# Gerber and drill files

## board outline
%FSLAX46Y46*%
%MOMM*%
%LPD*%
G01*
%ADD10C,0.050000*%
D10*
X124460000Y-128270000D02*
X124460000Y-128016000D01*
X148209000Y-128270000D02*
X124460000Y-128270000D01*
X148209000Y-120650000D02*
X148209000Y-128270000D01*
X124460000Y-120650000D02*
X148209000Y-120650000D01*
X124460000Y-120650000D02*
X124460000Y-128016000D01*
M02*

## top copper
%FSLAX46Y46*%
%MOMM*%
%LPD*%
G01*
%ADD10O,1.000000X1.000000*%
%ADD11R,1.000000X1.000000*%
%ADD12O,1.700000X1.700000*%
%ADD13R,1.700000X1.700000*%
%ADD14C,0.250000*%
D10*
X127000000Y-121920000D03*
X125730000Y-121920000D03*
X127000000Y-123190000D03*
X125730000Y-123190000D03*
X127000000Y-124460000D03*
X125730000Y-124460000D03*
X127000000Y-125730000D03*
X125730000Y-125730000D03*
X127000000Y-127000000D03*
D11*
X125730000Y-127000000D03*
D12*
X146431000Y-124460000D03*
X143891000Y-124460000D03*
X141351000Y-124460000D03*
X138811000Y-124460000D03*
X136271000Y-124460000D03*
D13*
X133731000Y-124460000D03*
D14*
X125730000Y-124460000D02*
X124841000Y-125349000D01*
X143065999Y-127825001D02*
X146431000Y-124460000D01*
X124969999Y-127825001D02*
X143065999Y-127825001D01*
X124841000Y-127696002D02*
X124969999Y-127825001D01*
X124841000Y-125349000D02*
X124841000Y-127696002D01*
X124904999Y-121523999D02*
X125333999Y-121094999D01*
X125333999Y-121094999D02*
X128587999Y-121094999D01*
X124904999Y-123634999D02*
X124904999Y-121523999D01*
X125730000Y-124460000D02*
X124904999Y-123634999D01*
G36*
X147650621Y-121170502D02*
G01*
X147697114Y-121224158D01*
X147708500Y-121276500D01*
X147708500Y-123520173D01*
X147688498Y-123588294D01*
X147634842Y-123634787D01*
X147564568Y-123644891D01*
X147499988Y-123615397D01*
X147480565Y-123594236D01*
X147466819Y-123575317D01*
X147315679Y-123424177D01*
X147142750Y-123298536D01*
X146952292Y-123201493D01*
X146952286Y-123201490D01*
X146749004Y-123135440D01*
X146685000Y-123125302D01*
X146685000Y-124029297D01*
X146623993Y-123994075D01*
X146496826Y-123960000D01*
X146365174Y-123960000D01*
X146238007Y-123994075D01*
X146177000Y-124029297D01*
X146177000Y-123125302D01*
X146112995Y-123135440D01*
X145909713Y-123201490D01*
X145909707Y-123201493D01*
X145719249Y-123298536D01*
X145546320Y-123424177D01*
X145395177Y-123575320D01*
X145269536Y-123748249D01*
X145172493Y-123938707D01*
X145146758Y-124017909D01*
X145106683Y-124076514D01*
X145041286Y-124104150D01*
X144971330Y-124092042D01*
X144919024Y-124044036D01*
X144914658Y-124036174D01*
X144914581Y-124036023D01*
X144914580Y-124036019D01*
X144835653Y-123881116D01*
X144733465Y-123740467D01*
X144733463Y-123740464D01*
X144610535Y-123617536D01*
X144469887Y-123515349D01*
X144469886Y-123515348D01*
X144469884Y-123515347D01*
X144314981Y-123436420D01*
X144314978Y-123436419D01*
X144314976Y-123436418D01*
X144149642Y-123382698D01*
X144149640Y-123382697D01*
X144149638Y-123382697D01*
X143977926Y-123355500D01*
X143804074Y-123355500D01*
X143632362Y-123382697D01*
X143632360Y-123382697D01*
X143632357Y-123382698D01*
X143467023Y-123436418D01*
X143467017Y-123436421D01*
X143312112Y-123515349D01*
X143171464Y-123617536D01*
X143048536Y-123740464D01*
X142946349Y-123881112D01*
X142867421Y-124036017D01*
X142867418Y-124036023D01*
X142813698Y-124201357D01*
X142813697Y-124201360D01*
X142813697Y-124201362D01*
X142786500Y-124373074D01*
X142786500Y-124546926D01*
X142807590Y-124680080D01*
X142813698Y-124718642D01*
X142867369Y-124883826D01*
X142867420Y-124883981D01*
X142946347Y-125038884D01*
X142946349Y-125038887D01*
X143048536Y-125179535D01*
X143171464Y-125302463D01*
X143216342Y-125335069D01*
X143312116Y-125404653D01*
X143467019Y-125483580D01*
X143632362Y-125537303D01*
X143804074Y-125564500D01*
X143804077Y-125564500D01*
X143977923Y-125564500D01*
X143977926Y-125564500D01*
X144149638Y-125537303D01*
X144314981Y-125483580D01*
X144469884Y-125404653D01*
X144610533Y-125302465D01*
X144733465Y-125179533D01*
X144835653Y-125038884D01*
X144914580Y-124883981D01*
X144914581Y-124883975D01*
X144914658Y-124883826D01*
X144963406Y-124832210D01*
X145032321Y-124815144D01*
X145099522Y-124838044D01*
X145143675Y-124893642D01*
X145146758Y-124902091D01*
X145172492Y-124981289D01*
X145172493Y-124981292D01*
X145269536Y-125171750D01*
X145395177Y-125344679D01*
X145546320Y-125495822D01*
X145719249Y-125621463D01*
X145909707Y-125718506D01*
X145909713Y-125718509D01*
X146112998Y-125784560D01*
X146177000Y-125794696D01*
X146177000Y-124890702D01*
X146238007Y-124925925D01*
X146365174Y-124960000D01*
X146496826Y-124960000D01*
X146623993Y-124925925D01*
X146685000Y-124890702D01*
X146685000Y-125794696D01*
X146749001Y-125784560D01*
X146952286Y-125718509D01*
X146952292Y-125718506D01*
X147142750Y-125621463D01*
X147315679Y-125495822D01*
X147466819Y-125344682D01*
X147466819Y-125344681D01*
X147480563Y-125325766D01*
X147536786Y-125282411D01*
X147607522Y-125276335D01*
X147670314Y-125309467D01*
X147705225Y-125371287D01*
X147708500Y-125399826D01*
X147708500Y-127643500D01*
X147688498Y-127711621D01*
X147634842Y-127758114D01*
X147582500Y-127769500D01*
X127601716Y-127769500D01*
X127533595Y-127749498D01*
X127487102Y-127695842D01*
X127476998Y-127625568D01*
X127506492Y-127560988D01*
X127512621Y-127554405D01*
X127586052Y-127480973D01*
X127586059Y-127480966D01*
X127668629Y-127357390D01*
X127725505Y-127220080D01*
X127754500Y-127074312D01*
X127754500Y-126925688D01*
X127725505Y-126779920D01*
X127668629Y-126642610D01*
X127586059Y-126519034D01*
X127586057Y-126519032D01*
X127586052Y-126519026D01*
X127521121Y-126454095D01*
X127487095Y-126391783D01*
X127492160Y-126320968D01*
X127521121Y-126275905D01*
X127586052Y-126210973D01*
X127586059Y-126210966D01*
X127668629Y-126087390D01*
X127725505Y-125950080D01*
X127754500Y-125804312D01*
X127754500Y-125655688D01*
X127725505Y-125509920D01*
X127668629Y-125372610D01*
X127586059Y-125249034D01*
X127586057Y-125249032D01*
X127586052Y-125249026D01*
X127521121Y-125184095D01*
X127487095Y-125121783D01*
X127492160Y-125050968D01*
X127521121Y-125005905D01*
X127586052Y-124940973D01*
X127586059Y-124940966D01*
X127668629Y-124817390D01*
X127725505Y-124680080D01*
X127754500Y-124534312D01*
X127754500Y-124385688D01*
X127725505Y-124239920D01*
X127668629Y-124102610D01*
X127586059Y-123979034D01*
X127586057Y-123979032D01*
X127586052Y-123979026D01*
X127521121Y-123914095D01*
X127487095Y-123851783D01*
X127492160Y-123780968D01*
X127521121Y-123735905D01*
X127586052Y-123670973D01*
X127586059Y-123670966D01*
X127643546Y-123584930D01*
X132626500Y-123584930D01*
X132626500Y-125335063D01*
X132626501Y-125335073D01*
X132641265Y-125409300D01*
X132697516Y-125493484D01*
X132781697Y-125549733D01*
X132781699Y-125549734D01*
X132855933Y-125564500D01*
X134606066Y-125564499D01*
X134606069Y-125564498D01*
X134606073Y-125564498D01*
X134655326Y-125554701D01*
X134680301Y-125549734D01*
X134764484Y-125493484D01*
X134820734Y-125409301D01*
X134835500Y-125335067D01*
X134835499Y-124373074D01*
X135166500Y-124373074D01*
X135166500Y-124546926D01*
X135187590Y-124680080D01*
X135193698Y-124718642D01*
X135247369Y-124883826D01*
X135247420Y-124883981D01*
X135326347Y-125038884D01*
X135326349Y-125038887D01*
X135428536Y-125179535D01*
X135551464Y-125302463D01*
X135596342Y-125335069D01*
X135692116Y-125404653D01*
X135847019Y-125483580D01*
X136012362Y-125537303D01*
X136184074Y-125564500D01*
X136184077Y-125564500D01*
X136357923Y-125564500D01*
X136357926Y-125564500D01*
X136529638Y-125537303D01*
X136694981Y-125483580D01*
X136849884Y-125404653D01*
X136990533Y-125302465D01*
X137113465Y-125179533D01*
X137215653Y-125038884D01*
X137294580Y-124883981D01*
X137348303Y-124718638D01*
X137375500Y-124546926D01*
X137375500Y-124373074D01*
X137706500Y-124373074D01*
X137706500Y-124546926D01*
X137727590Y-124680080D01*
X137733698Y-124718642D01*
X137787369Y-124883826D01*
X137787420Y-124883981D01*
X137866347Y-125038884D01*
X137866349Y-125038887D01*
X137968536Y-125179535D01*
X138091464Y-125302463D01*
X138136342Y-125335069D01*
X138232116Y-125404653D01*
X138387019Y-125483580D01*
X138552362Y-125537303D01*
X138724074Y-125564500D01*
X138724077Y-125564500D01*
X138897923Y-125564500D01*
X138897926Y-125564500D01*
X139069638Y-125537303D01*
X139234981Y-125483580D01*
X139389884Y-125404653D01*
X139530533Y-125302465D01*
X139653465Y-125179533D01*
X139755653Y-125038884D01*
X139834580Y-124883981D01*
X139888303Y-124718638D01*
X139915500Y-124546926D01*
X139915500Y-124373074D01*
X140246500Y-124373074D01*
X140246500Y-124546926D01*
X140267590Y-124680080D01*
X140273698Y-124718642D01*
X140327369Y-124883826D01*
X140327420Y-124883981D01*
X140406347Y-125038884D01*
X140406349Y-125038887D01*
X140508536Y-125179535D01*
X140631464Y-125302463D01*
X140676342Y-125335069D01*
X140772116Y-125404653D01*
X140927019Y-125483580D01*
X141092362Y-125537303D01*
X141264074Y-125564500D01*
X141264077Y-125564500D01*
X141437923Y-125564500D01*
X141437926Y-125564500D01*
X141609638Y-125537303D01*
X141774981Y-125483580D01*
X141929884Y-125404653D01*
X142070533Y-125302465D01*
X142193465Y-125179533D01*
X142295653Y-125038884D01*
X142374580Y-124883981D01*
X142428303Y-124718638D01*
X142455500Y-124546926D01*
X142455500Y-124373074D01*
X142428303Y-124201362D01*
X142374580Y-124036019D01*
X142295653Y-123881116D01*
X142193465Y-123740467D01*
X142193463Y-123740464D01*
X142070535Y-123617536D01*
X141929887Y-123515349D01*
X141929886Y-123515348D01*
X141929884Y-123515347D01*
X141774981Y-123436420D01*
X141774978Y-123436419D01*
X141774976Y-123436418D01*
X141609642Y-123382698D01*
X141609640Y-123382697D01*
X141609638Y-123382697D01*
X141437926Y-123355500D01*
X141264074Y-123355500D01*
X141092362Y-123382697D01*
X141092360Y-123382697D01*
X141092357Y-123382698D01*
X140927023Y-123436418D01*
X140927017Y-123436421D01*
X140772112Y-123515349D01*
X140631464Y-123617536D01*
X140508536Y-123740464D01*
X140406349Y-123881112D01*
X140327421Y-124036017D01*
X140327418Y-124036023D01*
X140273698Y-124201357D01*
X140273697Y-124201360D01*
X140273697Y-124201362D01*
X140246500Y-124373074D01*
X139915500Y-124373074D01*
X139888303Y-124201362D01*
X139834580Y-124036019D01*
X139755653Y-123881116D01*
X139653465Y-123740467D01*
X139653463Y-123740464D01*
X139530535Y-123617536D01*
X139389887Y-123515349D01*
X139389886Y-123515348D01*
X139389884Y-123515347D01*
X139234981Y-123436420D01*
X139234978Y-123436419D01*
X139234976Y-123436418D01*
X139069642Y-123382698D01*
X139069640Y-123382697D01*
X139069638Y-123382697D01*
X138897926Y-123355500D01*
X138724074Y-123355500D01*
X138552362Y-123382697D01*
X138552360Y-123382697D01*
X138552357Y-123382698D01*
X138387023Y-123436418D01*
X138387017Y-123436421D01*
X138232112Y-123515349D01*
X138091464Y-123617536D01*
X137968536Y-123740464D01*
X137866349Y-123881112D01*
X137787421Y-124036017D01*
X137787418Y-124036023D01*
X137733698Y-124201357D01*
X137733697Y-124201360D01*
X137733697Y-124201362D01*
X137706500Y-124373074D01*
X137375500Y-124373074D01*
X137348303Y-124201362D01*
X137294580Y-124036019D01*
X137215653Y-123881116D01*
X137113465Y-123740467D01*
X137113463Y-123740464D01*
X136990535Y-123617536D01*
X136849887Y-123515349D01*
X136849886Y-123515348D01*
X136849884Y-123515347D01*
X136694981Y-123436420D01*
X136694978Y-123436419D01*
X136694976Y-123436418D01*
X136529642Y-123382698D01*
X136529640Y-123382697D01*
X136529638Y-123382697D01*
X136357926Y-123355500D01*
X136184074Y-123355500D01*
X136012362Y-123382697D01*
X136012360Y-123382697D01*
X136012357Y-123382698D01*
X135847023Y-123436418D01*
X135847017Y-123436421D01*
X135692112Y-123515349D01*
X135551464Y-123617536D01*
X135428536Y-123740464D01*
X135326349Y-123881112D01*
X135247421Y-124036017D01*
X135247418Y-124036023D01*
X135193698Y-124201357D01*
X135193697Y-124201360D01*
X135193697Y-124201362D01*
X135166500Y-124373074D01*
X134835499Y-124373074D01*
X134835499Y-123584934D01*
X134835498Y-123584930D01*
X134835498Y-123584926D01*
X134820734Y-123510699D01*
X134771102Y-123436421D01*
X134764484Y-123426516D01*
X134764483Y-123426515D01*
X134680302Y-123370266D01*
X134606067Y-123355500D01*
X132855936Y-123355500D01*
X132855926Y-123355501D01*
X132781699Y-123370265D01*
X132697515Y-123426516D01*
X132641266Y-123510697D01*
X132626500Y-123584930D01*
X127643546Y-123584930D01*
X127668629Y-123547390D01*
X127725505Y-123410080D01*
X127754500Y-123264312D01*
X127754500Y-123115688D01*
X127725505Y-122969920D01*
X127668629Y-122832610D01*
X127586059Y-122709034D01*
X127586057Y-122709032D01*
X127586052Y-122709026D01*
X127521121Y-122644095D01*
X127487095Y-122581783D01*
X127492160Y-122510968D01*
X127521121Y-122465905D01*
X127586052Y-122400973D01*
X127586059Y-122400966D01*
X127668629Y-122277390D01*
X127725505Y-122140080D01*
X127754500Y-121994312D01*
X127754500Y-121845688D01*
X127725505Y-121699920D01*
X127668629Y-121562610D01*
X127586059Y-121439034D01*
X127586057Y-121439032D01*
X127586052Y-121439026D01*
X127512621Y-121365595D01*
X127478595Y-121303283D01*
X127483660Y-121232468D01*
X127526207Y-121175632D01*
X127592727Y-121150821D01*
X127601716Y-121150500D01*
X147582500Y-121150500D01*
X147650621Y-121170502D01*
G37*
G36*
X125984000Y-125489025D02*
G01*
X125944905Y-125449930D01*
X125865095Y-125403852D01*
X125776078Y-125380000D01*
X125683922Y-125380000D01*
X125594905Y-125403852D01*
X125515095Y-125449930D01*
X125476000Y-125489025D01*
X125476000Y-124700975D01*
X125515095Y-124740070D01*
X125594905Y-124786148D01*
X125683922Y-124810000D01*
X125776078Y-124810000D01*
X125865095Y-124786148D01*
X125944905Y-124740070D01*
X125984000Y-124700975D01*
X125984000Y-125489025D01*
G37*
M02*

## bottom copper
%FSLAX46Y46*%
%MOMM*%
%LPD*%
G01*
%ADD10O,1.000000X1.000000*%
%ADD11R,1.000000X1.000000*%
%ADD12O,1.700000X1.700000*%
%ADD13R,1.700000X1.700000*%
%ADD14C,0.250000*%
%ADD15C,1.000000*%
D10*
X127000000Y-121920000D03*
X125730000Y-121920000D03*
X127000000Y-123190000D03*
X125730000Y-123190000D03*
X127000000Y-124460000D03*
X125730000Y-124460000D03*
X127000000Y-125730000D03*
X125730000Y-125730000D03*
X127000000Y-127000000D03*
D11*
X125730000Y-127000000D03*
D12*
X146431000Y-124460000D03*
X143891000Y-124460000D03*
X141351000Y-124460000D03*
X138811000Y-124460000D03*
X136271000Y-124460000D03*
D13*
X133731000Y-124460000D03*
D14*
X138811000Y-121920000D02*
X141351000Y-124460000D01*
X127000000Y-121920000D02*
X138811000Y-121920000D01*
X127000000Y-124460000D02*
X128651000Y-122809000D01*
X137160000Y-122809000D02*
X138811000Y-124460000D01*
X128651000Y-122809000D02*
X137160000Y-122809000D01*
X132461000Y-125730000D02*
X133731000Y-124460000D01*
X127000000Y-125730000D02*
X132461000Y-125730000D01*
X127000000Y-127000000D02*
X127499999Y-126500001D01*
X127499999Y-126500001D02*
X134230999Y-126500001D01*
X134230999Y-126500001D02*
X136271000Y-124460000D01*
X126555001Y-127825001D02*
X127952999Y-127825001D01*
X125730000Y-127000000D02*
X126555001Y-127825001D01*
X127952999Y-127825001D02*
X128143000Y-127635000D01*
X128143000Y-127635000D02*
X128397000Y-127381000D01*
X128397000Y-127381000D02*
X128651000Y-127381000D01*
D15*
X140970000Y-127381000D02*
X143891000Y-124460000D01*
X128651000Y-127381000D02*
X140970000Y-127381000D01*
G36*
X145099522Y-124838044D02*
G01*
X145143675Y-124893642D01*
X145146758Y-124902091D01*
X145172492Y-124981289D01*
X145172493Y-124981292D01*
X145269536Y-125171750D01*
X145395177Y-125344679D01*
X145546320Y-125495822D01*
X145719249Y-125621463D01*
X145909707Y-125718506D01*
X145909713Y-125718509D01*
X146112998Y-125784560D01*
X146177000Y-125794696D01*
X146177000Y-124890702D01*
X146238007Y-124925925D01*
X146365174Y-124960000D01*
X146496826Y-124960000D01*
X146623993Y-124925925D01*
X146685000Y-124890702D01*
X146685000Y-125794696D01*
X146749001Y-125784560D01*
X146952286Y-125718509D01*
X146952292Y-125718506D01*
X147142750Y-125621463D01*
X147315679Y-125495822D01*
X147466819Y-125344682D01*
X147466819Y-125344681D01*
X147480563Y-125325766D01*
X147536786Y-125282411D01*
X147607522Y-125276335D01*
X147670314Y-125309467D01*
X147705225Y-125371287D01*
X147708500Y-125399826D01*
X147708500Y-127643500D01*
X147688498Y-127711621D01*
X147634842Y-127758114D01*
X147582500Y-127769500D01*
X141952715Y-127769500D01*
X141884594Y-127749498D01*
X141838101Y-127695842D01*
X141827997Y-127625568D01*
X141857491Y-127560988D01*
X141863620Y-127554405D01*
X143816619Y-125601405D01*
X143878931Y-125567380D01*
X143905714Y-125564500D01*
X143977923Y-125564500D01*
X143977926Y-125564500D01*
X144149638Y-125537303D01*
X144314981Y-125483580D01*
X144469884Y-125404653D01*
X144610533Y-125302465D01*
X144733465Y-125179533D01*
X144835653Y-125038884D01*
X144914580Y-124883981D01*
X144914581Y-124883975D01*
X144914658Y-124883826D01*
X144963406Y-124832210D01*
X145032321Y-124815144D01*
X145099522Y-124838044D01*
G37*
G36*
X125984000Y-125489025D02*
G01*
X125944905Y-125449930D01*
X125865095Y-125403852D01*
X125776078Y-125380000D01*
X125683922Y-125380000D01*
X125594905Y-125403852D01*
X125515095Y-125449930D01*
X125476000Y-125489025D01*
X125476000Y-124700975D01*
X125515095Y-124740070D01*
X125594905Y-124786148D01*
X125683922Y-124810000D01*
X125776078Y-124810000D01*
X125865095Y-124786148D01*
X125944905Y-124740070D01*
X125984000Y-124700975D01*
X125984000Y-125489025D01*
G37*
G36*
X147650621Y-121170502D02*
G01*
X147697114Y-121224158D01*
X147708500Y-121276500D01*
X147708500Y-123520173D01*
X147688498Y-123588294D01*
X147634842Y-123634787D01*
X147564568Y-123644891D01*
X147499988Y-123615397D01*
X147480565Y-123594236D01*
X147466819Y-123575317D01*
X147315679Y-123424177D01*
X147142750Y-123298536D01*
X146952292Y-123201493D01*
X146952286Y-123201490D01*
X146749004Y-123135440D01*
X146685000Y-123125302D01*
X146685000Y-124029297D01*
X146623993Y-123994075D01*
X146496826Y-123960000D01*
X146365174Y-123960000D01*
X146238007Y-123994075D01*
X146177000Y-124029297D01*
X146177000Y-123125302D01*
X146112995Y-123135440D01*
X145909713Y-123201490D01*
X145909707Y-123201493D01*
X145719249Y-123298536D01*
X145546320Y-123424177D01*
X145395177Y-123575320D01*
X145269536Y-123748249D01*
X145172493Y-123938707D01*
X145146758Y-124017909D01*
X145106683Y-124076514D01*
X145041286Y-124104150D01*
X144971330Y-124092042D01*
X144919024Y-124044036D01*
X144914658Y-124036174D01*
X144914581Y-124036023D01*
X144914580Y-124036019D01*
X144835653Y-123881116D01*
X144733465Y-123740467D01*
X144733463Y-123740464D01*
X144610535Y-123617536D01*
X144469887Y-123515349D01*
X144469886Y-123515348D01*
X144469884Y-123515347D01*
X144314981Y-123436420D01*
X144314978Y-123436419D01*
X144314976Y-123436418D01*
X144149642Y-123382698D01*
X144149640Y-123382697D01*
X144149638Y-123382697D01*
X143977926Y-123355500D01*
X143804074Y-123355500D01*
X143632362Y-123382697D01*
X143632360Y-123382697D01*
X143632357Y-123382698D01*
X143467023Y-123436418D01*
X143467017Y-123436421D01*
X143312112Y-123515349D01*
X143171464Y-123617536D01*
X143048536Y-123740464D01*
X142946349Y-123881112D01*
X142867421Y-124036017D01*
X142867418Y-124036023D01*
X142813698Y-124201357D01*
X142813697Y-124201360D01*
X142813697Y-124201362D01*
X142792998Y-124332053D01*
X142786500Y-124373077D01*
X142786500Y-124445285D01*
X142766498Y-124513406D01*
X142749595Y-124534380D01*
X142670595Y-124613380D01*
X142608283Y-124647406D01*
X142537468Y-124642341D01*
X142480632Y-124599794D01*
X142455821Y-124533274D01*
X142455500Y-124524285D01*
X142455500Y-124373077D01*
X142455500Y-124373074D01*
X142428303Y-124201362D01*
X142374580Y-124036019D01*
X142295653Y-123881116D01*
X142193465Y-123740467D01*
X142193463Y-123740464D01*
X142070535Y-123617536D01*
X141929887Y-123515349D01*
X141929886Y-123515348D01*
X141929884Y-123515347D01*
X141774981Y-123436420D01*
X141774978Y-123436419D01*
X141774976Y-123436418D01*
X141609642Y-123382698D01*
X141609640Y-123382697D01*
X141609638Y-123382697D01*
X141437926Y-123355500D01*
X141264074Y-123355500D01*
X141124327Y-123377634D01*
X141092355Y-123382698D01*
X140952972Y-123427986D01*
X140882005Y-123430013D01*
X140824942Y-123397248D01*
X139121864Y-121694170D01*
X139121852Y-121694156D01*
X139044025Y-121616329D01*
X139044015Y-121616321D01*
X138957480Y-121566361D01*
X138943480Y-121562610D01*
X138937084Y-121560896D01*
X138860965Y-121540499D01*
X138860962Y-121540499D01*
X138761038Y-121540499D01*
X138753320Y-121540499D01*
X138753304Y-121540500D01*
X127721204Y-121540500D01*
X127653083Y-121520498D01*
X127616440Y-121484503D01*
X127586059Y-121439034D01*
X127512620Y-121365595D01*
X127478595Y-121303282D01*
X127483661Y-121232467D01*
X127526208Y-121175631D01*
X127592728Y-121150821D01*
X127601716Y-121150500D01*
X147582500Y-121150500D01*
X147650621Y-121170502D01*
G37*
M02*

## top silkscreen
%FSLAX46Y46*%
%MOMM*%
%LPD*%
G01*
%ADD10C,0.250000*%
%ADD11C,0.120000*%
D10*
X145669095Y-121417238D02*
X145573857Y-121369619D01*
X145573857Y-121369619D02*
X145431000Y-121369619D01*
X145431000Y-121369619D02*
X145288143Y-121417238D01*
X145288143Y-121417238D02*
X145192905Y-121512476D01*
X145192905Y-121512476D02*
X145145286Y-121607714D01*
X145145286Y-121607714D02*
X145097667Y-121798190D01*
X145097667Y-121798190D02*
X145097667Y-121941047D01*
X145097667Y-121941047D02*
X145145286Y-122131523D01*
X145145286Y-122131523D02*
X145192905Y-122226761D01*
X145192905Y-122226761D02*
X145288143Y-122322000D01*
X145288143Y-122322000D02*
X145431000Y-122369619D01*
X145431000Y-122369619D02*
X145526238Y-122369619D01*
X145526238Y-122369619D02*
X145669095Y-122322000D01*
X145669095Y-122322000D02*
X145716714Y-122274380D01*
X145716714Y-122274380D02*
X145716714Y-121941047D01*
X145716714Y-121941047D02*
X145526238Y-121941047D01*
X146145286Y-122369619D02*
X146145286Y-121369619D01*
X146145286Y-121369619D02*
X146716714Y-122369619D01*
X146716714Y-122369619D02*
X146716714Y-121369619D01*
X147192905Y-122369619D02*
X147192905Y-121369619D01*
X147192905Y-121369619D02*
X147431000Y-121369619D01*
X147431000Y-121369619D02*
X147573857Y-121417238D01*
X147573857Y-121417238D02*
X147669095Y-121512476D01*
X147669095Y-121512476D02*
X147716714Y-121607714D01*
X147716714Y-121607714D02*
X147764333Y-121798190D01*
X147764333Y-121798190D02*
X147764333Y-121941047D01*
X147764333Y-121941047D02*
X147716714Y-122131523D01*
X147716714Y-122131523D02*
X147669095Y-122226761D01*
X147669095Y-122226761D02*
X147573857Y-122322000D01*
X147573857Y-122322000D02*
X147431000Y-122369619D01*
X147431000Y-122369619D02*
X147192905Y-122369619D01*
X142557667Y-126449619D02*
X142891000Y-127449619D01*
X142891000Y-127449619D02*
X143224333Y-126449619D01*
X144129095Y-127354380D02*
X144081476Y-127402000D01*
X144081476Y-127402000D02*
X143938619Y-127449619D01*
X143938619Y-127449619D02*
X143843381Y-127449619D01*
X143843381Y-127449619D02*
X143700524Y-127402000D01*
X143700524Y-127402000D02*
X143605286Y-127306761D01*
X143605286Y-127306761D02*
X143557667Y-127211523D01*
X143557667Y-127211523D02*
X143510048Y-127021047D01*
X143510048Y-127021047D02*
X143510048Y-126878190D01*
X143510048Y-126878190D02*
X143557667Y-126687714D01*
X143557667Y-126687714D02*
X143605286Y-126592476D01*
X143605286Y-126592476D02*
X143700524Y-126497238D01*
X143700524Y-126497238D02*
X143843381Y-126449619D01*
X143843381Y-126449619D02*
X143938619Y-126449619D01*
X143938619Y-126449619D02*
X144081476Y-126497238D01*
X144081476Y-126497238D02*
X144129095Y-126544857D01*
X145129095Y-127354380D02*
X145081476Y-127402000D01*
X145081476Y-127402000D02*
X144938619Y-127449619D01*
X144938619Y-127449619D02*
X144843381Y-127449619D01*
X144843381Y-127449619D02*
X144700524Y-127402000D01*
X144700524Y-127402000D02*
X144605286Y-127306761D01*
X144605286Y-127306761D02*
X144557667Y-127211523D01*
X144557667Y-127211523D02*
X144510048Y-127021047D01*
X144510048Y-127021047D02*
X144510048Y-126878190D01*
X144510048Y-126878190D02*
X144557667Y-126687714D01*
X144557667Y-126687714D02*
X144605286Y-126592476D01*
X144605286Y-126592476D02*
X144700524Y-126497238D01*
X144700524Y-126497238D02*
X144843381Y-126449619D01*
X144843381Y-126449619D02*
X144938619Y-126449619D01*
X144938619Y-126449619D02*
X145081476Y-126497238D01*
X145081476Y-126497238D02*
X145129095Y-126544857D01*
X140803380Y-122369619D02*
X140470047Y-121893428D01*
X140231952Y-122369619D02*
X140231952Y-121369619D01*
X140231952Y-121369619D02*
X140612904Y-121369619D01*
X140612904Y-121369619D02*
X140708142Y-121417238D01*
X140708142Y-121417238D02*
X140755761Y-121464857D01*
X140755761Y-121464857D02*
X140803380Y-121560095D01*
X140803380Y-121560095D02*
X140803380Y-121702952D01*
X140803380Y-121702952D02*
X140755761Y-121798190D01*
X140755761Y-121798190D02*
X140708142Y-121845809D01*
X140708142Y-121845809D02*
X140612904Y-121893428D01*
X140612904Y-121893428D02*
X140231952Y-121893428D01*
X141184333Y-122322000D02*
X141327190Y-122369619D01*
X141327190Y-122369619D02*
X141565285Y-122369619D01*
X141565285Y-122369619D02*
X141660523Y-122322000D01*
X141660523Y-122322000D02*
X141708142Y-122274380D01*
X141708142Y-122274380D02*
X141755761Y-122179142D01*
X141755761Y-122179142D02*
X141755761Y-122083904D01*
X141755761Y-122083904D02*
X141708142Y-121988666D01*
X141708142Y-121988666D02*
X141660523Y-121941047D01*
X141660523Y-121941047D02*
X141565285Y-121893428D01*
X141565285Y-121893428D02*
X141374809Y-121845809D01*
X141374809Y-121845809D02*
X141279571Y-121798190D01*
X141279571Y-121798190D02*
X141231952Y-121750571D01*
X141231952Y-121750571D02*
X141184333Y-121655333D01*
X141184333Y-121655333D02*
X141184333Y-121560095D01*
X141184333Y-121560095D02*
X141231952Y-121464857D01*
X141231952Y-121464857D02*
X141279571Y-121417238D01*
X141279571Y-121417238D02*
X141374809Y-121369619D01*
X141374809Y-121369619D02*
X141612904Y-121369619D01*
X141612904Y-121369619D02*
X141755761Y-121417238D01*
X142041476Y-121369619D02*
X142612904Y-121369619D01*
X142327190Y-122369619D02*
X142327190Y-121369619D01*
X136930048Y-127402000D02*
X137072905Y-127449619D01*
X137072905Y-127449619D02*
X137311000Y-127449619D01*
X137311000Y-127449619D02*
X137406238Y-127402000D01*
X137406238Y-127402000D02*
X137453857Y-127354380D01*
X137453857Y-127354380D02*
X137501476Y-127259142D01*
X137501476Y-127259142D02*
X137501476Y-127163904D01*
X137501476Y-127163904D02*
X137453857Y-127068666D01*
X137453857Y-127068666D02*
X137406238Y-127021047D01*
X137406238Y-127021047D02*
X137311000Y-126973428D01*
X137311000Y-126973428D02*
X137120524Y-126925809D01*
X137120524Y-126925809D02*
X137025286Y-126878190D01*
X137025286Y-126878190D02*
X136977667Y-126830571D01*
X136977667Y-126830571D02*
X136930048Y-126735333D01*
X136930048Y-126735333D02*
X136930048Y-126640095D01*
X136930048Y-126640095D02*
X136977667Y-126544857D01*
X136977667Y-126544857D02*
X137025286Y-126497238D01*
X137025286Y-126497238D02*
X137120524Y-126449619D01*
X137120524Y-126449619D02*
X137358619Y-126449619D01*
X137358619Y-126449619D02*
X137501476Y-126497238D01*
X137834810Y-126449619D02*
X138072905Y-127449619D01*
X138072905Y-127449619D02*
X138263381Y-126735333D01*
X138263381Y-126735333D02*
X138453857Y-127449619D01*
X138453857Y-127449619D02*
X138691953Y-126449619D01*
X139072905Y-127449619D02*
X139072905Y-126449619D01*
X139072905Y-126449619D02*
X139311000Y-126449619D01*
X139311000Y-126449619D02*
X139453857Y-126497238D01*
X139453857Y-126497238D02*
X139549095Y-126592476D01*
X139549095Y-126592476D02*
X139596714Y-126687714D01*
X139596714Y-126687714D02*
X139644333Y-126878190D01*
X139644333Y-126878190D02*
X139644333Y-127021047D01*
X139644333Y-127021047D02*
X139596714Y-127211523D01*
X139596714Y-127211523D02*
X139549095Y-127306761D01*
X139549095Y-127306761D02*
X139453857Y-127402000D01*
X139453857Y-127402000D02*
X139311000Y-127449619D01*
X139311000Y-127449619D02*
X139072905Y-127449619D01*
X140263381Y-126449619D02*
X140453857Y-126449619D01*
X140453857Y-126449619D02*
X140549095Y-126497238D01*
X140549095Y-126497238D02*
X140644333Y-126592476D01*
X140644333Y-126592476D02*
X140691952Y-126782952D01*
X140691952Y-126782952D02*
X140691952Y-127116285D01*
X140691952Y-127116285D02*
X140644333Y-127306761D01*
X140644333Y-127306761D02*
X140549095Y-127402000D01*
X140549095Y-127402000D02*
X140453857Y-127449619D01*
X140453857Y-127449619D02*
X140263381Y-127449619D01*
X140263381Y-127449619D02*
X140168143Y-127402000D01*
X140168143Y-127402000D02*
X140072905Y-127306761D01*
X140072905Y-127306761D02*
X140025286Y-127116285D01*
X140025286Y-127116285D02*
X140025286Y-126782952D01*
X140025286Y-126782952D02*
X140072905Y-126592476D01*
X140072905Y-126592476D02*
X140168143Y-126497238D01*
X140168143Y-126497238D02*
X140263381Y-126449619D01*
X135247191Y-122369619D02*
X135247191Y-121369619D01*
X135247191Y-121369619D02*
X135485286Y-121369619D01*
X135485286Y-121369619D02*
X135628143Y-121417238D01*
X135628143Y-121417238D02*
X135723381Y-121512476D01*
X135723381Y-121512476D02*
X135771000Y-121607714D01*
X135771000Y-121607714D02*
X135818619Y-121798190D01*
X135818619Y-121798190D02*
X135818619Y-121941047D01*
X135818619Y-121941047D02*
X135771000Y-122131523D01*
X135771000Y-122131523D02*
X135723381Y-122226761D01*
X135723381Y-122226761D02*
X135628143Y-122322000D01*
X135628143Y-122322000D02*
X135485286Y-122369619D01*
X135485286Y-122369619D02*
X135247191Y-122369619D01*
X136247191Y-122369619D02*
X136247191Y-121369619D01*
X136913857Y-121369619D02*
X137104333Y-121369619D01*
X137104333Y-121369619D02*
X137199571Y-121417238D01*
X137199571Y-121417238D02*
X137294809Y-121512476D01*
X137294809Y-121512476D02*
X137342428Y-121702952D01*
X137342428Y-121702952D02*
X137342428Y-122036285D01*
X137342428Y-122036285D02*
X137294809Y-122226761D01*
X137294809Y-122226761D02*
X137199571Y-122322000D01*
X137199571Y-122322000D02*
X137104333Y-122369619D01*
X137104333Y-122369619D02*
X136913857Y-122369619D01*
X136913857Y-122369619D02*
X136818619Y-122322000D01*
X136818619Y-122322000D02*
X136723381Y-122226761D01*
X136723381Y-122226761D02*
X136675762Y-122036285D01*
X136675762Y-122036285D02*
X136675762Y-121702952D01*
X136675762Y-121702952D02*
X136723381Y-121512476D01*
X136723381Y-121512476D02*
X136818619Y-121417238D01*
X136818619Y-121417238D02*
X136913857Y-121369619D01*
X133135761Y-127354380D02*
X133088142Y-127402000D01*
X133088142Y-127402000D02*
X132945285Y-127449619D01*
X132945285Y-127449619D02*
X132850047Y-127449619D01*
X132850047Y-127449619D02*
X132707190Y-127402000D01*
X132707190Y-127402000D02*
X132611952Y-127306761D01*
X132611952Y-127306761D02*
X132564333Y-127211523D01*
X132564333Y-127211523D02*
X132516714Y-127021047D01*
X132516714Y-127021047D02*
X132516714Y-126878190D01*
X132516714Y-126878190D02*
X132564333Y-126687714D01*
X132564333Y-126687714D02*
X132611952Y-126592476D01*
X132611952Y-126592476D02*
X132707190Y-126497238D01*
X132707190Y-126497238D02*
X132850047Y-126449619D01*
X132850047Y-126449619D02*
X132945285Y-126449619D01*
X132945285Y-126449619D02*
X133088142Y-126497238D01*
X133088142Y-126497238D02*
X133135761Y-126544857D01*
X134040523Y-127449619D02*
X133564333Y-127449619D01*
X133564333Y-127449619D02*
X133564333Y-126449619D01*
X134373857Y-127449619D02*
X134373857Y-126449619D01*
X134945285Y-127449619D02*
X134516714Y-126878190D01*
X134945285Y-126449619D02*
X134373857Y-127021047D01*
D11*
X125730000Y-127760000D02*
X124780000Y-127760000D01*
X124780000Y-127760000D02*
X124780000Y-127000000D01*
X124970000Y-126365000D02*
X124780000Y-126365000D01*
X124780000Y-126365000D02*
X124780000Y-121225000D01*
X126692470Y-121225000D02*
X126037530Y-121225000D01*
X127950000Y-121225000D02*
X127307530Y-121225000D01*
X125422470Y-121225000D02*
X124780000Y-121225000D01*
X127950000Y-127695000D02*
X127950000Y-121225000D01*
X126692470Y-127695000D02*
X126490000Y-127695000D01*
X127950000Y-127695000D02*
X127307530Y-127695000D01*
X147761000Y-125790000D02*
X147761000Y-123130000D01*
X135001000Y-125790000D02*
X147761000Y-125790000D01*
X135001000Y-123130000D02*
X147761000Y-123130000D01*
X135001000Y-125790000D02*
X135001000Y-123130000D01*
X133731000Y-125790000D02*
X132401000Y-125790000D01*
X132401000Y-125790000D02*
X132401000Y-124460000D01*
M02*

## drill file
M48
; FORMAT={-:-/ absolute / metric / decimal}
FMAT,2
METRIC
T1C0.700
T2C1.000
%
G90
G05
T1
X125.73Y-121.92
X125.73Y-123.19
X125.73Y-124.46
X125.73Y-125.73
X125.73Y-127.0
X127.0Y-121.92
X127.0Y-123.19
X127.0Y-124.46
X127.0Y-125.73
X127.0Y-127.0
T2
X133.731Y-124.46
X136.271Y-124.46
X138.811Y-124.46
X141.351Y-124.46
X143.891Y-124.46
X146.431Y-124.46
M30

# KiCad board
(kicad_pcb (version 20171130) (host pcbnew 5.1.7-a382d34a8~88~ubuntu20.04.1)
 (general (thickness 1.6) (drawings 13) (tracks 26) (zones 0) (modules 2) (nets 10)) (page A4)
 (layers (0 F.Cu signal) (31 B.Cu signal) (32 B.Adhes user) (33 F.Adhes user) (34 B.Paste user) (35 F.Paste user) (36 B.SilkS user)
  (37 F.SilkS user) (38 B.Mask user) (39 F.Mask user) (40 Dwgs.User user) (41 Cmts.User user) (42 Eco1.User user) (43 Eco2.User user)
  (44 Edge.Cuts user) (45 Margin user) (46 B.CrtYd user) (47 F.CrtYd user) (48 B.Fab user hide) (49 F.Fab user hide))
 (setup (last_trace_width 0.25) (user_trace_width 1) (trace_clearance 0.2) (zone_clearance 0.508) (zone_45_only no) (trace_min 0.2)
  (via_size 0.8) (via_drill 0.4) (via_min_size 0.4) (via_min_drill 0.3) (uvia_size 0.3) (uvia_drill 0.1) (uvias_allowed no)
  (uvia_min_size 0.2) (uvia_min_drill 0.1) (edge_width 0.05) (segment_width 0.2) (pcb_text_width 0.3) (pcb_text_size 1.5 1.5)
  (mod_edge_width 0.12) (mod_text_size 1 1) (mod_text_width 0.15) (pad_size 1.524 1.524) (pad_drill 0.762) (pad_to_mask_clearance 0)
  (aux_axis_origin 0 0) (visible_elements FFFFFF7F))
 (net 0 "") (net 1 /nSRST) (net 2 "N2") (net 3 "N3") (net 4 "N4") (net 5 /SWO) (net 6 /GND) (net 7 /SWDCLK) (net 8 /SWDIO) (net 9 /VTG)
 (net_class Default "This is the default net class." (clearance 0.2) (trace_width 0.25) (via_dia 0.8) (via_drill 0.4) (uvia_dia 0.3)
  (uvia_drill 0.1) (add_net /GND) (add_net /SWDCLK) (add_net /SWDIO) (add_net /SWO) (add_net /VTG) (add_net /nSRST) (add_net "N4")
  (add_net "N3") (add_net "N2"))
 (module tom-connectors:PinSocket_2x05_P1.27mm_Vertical (layer F.Cu) (at 125.73 127 180)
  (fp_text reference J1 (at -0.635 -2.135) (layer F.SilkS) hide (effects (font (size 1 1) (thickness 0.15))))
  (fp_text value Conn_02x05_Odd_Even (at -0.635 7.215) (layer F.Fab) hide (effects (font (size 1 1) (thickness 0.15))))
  (fp_line (start 0 -0.76) (end 0.95 -0.76) (layer F.SilkS) (width 0.12))
  (fp_line (start 0.95 -0.76) (end 0.95 0) (layer F.SilkS) (width 0.12))
  (fp_line (start 0.76 0.635) (end 0.95 0.635) (layer F.SilkS) (width 0.12))
  (fp_line (start 0.95 0.635) (end 0.95 5.775) (layer F.SilkS) (width 0.12))
  (fp_line (start -0.96247 5.775) (end -0.30753 5.775) (layer F.SilkS) (width 0.12))
  (fp_line (start -2.22 5.775) (end -1.57753 5.775) (layer F.SilkS) (width 0.12))
  (fp_line (start 0.30753 5.775) (end 0.95 5.775) (layer F.SilkS) (width 0.12))
  (fp_line (start -2.22 -0.695) (end -2.22 5.775) (layer F.SilkS) (width 0.12))
  (fp_line (start -0.96247 -0.695) (end -0.76 -0.695) (layer F.SilkS) (width 0.12))
  (fp_line (start -2.22 -0.695) (end -1.57753 -0.695) (layer F.SilkS) (width 0.12))
  (pad 10 thru_hole oval (at -1.27 5.08 180) (size 1 1) (drill 0.7) (layers *.Cu *.Mask) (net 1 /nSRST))
  (pad 9 thru_hole oval (at 0 5.08 180) (size 1 1) (drill 0.7) (layers *.Cu *.Mask) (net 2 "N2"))
  (pad 8 thru_hole oval (at -1.27 3.81 180) (size 1 1) (drill 0.7) (layers *.Cu *.Mask) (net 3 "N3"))
  (pad 7 thru_hole oval (at 0 3.81 180) (size 1 1) (drill 0.7) (layers *.Cu *.Mask) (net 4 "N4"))
  (pad 6 thru_hole oval (at -1.27 2.54 180) (size 1 1) (drill 0.7) (layers *.Cu *.Mask) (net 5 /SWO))
  (pad 5 thru_hole oval (at 0 2.54 180) (size 1 1) (drill 0.7) (layers *.Cu *.Mask) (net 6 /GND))
  (pad 4 thru_hole oval (at -1.27 1.27 180) (size 1 1) (drill 0.7) (layers *.Cu *.Mask) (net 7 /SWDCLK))
  (pad 3 thru_hole oval (at 0 1.27 180) (size 1 1) (drill 0.7) (layers *.Cu *.Mask) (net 6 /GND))
  (pad 2 thru_hole oval (at -1.27 0 180) (size 1 1) (drill 0.7) (layers *.Cu *.Mask) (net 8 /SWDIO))
  (pad 1 thru_hole rect (at 0 0 180) (size 1 1) (drill 0.7) (layers *.Cu *.Mask) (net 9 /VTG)))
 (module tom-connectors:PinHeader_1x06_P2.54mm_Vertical (layer F.Cu) (at 133.731 124.46 90)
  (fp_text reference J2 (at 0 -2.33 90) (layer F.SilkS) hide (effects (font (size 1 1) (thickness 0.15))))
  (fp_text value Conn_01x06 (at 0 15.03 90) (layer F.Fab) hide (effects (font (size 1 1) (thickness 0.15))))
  (fp_line (start -1.33 14.03) (end 1.33 14.03) (layer F.SilkS) (width 0.12))
  (fp_line (start -1.33 1.27) (end -1.33 14.03) (layer F.SilkS) (width 0.12))
  (fp_line (start 1.33 1.27) (end 1.33 14.03) (layer F.SilkS) (width 0.12))
  (fp_line (start -1.33 1.27) (end 1.33 1.27) (layer F.SilkS) (width 0.12))
  (fp_line (start -1.33 0) (end -1.33 -1.33) (layer F.SilkS) (width 0.12))
  (fp_line (start -1.33 -1.33) (end 0 -1.33) (layer F.SilkS) (width 0.12))
  (pad 6 thru_hole oval (at 0 12.7 90) (size 1.7 1.7) (drill 1) (layers *.Cu *.Mask) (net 6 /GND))
  (pad 5 thru_hole oval (at 0 10.16 90) (size 1.7 1.7) (drill 1) (layers *.Cu *.Mask) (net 9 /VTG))
  (pad 4 thru_hole oval (at 0 7.62 90) (size 1.7 1.7) (drill 1) (layers *.Cu *.Mask) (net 1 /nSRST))
  (pad 3 thru_hole oval (at 0 5.08 90) (size 1.7 1.7) (drill 1) (layers *.Cu *.Mask) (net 5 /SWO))
  (pad 2 thru_hole oval (at 0 2.54 90) (size 1.7 1.7) (drill 1) (layers *.Cu *.Mask) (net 8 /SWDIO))
  (pad 1 thru_hole rect (at 0 0 90) (size 1.7 1.7) (drill 1) (layers *.Cu *.Mask) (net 7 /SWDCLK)))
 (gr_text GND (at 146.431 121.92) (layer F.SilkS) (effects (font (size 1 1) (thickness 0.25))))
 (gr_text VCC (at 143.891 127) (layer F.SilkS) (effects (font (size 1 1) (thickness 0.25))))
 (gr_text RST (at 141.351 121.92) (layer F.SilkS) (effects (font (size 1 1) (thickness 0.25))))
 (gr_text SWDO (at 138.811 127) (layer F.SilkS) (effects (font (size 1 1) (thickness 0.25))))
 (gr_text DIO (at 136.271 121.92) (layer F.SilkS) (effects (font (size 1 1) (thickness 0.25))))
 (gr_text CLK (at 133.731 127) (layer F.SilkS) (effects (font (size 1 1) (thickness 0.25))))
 (gr_line (start 124.46 128.27) (end 124.46 128.016) (layer Edge.Cuts) (width 0.05))
 (gr_line (start 148.209 128.27) (end 124.46 128.27) (layer Edge.Cuts) (width 0.05))
 (gr_line (start 148.209 120.65) (end 148.209 128.27) (layer Edge.Cuts) (width 0.05))
 (gr_line (start 124.46 120.65) (end 148.209 120.65) (layer Edge.Cuts) (width 0.05))
 (gr_line (start 124.46 120.65) (end 124.46 128.016) (layer Edge.Cuts) (width 0.05))
 (segment (start 138.811 121.92) (end 141.351 124.46) (width 0.25) (layer B.Cu) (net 1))
 (segment (start 127 121.92) (end 138.811 121.92) (width 0.25) (layer B.Cu) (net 1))
 (segment (start 125.73 124.46) (end 124.841 125.349) (width 0.25) (layer F.Cu) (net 6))
 (segment (start 143.065999 127.825001) (end 146.431 124.46) (width 0.25) (layer F.Cu) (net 6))
 (segment (start 124.969999 127.825001) (end 143.065999 127.825001) (width 0.25) (layer F.Cu) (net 6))
 (segment (start 124.841 127.696002) (end 124.969999 127.825001) (width 0.25) (layer F.Cu) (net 6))
 (segment (start 124.841 125.349) (end 124.841 127.696002) (width 0.25) (layer F.Cu) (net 6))
 (segment (start 124.904999 121.523999) (end 125.333999 121.094999) (width 0.25) (layer F.Cu) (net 6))
 (segment (start 125.333999 121.094999) (end 128.587999 121.094999) (width 0.25) (layer F.Cu) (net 6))
 (segment (start 124.904999 123.634999) (end 124.904999 121.523999) (width 0.25) (layer F.Cu) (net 6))
 (segment (start 125.73 124.46) (end 124.904999 123.634999) (width 0.25) (layer F.Cu) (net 6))
 (segment (start 127 124.46) (end 128.651 122.809) (width 0.25) (layer B.Cu) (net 5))
 (segment (start 137.16 122.809) (end 138.811 124.46) (width 0.25) (layer B.Cu) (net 5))
 (segment (start 128.651 122.809) (end 137.16 122.809) (width 0.25) (layer B.Cu) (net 5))
 (segment (start 132.461 125.73) (end 133.731 124.46) (width 0.25) (layer B.Cu) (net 7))
 (segment (start 127 125.73) (end 132.461 125.73) (width 0.25) (layer B.Cu) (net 7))
 (segment (start 127 127) (end 127.499999 126.500001) (width 0.25) (layer B.Cu) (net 8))
 (segment (start 127.499999 126.500001) (end 134.230999 126.500001) (width 0.25) (layer B.Cu) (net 8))
 (segment (start 134.230999 126.500001) (end 136.271 124.46) (width 0.25) (layer B.Cu) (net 8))
 (segment (start 126.555001 127.825001) (end 127.952999 127.825001) (width 0.25) (layer B.Cu) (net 9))
 (segment (start 125.73 127) (end 126.555001 127.825001) (width 0.25) (layer B.Cu) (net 9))
 (segment (start 127.952999 127.825001) (end 128.143 127.635) (width 0.25) (layer B.Cu) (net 9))
 (segment (start 128.143 127.635) (end 128.397 127.381) (width 0.25) (layer B.Cu) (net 9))
 (segment (start 128.397 127.381) (end 128.651 127.381) (width 0.25) (layer B.Cu) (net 9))
 (segment (start 140.97 127.381) (end 143.891 124.46) (width 1) (layer B.Cu) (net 9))
 (segment (start 128.651 127.381) (end 140.97 127.381) (width 1) (layer B.Cu) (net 9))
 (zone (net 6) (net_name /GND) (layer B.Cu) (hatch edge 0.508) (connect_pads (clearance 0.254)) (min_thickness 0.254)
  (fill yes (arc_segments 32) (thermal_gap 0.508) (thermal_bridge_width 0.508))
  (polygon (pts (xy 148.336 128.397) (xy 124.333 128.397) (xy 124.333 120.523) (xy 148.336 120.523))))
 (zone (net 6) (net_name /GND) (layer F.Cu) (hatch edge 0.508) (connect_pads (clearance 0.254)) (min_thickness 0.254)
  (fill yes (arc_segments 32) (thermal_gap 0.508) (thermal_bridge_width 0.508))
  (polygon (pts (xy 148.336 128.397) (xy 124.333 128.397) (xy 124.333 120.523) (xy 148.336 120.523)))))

